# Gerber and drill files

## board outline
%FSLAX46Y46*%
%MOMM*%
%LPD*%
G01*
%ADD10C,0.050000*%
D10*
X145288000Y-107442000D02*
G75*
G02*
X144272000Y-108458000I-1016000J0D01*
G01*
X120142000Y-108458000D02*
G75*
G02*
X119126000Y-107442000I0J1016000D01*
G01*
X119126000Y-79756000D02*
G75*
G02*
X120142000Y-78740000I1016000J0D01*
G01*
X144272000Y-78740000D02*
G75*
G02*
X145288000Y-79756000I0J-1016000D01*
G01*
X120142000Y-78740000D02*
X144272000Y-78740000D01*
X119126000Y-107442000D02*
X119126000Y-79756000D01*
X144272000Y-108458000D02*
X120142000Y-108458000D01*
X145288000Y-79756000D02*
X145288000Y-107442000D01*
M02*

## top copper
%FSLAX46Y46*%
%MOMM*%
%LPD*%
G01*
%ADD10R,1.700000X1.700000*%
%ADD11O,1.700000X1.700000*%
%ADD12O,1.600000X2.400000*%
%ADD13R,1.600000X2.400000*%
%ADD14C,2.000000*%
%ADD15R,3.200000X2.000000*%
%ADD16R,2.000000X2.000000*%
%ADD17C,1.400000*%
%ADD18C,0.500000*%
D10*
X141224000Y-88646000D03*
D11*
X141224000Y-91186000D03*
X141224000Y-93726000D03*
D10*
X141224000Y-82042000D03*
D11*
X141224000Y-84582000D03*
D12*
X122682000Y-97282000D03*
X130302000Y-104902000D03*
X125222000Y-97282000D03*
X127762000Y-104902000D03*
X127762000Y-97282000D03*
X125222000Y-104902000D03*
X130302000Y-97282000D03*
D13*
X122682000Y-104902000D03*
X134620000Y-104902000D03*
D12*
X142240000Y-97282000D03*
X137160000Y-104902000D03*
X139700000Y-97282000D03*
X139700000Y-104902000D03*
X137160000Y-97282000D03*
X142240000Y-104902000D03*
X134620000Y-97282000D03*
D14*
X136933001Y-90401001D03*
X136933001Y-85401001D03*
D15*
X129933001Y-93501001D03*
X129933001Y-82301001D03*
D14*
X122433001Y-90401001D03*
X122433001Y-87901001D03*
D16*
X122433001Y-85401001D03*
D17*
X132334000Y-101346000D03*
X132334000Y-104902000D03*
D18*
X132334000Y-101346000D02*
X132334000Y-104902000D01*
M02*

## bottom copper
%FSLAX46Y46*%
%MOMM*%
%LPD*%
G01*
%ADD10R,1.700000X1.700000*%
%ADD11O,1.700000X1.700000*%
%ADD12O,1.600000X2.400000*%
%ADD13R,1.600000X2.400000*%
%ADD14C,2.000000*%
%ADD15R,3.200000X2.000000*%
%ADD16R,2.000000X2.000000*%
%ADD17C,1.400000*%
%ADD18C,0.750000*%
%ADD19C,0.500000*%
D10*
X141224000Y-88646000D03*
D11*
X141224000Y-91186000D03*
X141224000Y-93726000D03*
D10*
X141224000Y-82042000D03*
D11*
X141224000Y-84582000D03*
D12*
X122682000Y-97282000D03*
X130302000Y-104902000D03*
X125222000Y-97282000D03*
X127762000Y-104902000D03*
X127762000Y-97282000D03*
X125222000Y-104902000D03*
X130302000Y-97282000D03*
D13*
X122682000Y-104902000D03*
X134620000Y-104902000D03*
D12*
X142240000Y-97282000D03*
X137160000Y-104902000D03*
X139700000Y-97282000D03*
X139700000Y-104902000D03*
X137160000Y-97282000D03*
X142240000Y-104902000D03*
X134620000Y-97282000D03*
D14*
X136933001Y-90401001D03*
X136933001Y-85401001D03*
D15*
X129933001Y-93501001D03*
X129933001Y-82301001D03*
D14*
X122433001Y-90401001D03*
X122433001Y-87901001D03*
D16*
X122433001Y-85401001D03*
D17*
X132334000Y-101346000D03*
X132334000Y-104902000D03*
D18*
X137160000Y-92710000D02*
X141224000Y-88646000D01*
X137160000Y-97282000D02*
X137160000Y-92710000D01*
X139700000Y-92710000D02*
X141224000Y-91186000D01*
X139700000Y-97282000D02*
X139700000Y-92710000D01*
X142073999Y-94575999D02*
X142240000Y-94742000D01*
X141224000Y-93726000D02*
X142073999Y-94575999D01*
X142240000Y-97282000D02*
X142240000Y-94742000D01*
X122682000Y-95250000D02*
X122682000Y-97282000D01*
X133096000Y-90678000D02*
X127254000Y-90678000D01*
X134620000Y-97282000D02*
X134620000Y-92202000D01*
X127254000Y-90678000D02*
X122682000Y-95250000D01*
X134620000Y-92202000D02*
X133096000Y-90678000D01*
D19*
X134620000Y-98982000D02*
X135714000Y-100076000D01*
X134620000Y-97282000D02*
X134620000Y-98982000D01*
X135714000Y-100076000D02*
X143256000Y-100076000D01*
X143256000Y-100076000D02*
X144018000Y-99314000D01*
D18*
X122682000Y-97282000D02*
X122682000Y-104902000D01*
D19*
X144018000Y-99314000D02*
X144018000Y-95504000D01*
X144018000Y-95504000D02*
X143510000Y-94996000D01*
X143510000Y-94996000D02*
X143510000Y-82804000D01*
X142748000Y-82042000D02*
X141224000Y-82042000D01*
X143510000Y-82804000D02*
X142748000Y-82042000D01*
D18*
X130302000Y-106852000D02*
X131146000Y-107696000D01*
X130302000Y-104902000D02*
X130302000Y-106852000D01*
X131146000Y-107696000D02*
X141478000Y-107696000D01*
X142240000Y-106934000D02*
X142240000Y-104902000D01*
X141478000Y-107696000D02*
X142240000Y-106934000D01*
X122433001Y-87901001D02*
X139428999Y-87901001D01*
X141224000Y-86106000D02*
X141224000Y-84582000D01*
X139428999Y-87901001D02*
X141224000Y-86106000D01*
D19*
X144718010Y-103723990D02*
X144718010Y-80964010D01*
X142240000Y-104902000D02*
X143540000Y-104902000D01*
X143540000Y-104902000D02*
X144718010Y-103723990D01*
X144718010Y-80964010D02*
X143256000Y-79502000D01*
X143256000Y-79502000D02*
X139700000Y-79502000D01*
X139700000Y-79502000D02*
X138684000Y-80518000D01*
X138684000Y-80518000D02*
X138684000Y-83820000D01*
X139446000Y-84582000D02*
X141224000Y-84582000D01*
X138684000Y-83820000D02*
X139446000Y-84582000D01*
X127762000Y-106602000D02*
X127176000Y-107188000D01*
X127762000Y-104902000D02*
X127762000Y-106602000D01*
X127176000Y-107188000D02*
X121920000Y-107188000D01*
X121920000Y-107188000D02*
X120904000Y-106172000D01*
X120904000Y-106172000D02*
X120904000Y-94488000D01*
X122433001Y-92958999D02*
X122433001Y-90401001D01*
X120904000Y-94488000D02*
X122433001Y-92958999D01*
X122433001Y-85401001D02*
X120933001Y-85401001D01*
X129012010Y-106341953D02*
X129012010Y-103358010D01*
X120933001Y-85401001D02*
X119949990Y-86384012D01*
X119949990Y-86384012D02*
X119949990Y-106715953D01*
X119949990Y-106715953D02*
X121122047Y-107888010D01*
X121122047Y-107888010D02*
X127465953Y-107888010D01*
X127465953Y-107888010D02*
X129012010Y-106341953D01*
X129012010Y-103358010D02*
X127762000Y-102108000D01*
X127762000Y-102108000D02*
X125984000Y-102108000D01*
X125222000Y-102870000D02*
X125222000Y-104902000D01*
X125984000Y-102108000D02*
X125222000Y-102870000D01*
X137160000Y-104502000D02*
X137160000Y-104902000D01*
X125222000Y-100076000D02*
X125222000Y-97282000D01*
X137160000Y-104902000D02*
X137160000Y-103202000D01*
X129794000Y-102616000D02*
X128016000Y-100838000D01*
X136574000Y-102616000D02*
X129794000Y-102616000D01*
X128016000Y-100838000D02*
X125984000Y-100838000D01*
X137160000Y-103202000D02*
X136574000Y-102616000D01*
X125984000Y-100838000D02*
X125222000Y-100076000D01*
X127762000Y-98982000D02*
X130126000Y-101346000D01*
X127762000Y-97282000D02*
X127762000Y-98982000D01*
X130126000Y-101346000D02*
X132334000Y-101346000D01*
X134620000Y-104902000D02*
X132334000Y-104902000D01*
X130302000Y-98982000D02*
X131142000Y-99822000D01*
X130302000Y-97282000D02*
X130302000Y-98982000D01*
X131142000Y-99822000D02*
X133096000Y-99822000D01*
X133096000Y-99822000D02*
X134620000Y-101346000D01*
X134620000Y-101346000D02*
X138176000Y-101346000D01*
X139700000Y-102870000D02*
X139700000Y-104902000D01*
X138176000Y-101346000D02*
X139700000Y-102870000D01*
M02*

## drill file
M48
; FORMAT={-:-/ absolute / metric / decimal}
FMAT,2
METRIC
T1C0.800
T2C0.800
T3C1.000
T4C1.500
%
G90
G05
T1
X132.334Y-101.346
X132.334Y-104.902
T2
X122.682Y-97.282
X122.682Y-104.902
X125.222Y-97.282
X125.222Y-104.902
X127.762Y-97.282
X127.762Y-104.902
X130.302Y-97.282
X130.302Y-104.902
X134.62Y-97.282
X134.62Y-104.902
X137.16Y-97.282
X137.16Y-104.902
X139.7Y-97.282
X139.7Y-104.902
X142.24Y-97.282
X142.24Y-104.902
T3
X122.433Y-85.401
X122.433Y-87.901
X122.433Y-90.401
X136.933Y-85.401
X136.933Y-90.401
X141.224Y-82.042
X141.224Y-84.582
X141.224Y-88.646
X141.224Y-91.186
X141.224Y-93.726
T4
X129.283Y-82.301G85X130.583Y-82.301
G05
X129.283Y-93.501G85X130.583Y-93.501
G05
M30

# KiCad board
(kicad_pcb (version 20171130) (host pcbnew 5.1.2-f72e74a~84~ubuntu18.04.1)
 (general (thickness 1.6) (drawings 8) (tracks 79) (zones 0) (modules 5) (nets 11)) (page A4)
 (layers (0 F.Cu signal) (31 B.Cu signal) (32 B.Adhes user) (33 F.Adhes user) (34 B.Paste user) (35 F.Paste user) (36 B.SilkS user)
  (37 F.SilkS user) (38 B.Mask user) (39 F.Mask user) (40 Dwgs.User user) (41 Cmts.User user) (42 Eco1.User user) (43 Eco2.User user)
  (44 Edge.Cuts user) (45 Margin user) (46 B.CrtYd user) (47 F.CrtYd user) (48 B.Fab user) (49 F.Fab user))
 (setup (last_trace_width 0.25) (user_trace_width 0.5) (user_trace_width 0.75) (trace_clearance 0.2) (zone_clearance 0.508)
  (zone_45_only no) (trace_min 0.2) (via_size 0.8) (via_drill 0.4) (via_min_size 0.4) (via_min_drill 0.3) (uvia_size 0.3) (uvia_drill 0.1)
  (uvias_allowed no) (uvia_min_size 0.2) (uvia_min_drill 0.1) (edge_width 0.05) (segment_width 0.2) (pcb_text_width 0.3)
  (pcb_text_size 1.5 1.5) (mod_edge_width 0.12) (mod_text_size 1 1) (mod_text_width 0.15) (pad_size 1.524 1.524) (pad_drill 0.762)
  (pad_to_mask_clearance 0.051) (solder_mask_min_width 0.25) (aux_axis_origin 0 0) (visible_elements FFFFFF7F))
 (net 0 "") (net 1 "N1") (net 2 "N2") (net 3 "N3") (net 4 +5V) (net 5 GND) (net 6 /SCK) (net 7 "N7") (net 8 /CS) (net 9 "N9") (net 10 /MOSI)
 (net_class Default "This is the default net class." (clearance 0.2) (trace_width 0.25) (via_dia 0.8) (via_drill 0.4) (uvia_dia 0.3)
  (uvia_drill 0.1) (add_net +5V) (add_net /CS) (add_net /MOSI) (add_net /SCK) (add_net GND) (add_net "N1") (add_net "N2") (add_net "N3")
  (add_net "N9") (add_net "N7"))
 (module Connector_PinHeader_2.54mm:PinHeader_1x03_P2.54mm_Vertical (layer F.Cu) (at 141.224 88.646)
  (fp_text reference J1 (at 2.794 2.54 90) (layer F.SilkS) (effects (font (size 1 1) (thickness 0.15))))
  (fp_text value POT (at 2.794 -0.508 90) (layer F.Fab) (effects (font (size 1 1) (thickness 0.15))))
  (pad 1 thru_hole rect (at 0 0) (size 1.7 1.7) (drill 1) (layers *.Cu *.Mask) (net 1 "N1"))
  (pad 2 thru_hole oval (at 0 2.54) (size 1.7 1.7) (drill 1) (layers *.Cu *.Mask) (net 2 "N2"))
  (pad 3 thru_hole oval (at 0 5.08) (size 1.7 1.7) (drill 1) (layers *.Cu *.Mask) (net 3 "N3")))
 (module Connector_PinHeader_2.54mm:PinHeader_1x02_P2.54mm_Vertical (layer F.Cu) (at 141.224 82.042)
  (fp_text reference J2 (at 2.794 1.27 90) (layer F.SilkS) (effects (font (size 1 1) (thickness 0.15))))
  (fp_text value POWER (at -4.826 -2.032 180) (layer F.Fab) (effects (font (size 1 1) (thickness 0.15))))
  (pad 1 thru_hole rect (at 0 0) (size 1.7 1.7) (drill 1) (layers *.Cu *.Mask) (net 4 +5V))
  (pad 2 thru_hole oval (at 0 2.54) (size 1.7 1.7) (drill 1) (layers *.Cu *.Mask) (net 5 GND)))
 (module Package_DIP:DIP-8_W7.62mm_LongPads (layer F.Cu) (at 122.682 104.902 90)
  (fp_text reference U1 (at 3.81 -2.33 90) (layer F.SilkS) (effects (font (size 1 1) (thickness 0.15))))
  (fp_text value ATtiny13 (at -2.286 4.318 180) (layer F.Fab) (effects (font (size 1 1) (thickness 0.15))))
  (pad 8 thru_hole oval (at 7.62 0 90) (size 2.4 1.6) (drill 0.8) (layers *.Cu *.Mask) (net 4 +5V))
  (pad 4 thru_hole oval (at 0 7.62 90) (size 2.4 1.6) (drill 0.8) (layers *.Cu *.Mask) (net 5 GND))
  (pad 7 thru_hole oval (at 7.62 2.54 90) (size 2.4 1.6) (drill 0.8) (layers *.Cu *.Mask) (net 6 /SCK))
  (pad 3 thru_hole oval (at 0 5.08 90) (size 2.4 1.6) (drill 0.8) (layers *.Cu *.Mask) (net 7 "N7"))
  (pad 6 thru_hole oval (at 7.62 5.08 90) (size 2.4 1.6) (drill 0.8) (layers *.Cu *.Mask) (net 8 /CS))
  (pad 2 thru_hole oval (at 0 2.54 90) (size 2.4 1.6) (drill 0.8) (layers *.Cu *.Mask) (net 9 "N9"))
  (pad 5 thru_hole oval (at 7.62 7.62 90) (size 2.4 1.6) (drill 0.8) (layers *.Cu *.Mask) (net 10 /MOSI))
  (pad 1 thru_hole rect (at 0 0 90) (size 2.4 1.6) (drill 0.8) (layers *.Cu *.Mask) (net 4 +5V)))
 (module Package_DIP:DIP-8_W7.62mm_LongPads (layer F.Cu) (at 134.62 104.902 90)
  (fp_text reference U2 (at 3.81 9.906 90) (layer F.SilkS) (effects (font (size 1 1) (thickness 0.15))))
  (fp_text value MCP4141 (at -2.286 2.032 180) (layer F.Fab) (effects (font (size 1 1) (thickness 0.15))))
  (pad 1 thru_hole rect (at 0 0 90) (size 2.4 1.6) (drill 0.8) (layers *.Cu *.Mask) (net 8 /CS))
  (pad 5 thru_hole oval (at 7.62 7.62 90) (size 2.4 1.6) (drill 0.8) (layers *.Cu *.Mask) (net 3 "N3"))
  (pad 2 thru_hole oval (at 0 2.54 90) (size 2.4 1.6) (drill 0.8) (layers *.Cu *.Mask) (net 6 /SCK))
  (pad 6 thru_hole oval (at 7.62 5.08 90) (size 2.4 1.6) (drill 0.8) (layers *.Cu *.Mask) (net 2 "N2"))
  (pad 3 thru_hole oval (at 0 5.08 90) (size 2.4 1.6) (drill 0.8) (layers *.Cu *.Mask) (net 10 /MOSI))
  (pad 7 thru_hole oval (at 7.62 2.54 90) (size 2.4 1.6) (drill 0.8) (layers *.Cu *.Mask) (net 1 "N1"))
  (pad 4 thru_hole oval (at 0 7.62 90) (size 2.4 1.6) (drill 0.8) (layers *.Cu *.Mask) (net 5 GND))
  (pad 8 thru_hole oval (at 7.62 0 90) (size 2.4 1.6) (drill 0.8) (layers *.Cu *.Mask) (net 4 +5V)))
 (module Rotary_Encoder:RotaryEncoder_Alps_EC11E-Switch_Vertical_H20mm (layer F.Cu) (at 122.433001 85.401001)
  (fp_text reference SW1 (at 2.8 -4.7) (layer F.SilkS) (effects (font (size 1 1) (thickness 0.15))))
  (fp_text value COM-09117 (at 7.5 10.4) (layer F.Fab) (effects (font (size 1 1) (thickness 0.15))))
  (pad S1 thru_hole circle (at 14.5 5) (size 2 2) (drill 1) (layers *.Cu *.Mask))
  (pad S2 thru_hole circle (at 14.5 0) (size 2 2) (drill 1) (layers *.Cu *.Mask))
  (pad MP thru_hole rect (at 7.5 8.1) (size 3.2 2) (drill oval 2.8 1.5) (layers *.Cu *.Mask))
  (pad MP thru_hole rect (at 7.5 -3.1) (size 3.2 2) (drill oval 2.8 1.5) (layers *.Cu *.Mask))
  (pad B thru_hole circle (at 0 5) (size 2 2) (drill 1) (layers *.Cu *.Mask) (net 7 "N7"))
  (pad C thru_hole circle (at 0 2.5) (size 2 2) (drill 1) (layers *.Cu *.Mask) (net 5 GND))
  (pad A thru_hole rect (at 0 0) (size 2 2) (drill 1) (layers *.Cu *.Mask) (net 9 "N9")))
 (gr_arc (start 144.272 107.442) (end 144.272 108.458) (angle -90) (layer Edge.Cuts) (width 0.05))
 (gr_arc (start 120.142 107.442) (end 119.126 107.442) (angle -90) (layer Edge.Cuts) (width 0.05))
 (gr_arc (start 120.142 79.756) (end 120.142 78.74) (angle -90) (layer Edge.Cuts) (width 0.05))
 (gr_arc (start 144.272 79.756) (end 145.288 79.756) (angle -90) (layer Edge.Cuts) (width 0.05))
 (gr_line (start 120.142 78.74) (end 144.272 78.74) (layer Edge.Cuts) (width 0.05))
 (gr_line (start 119.126 107.442) (end 119.126 79.756) (layer Edge.Cuts) (width 0.05))
 (gr_line (start 144.272 108.458) (end 120.142 108.458) (layer Edge.Cuts) (width 0.05))
 (gr_line (start 145.288 79.756) (end 145.288 107.442) (layer Edge.Cuts) (width 0.05))
 (segment (start 137.16 92.71) (end 141.224 88.646) (width 0.75) (layer B.Cu) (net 1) (status 20))
 (segment (start 137.16 97.282) (end 137.16 92.71) (width 0.75) (layer B.Cu) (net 1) (status 10))
 (segment (start 139.7 92.71) (end 141.224 91.186) (width 0.75) (layer B.Cu) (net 2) (status 20))
 (segment (start 139.7 97.282) (end 139.7 92.71) (width 0.75) (layer B.Cu) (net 2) (status 10))
 (segment (start 142.073999 94.575999) (end 142.24 94.742) (width 0.75) (layer B.Cu) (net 3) (status 10))
 (segment (start 141.224 93.726) (end 142.073999 94.575999) (width 0.75) (layer B.Cu) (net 3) (status 30))
 (segment (start 142.24 97.282) (end 142.24 94.742) (width 0.75) (layer B.Cu) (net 3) (status 10))
 (segment (start 122.682 95.25) (end 122.682 97.282) (width 0.75) (layer B.Cu) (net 4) (status 20))
 (segment (start 133.096 90.678) (end 127.254 90.678) (width 0.75) (layer B.Cu) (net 4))
 (segment (start 134.62 97.282) (end 134.62 92.202) (width 0.75) (layer B.Cu) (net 4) (status 10))
 (segment (start 127.254 90.678) (end 122.682 95.25) (width 0.75) (layer B.Cu) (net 4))
 (segment (start 134.62 92.202) (end 133.096 90.678) (width 0.75) (layer B.Cu) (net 4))
 (segment (start 134.62 98.982) (end 135.714 100.076) (width 0.5) (layer B.Cu) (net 4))
 (segment (start 134.62 97.282) (end 134.62 98.982) (width 0.5) (layer B.Cu) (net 4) (status 10))
 (segment (start 135.714 100.076) (end 143.256 100.076) (width 0.5) (layer B.Cu) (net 4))
 (segment (start 143.256 100.076) (end 144.018 99.314) (width 0.5) (layer B.Cu) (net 4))
 (segment (start 122.682 97.282) (end 122.682 104.902) (width 0.75) (layer B.Cu) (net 4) (status 30))
 (segment (start 144.018 99.314) (end 144.018 95.504) (width 0.5) (layer B.Cu) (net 4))
 (segment (start 144.018 95.504) (end 143.51 94.996) (width 0.5) (layer B.Cu) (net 4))
 (segment (start 143.51 94.996) (end 143.51 82.804) (width 0.5) (layer B.Cu) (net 4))
 (segment (start 142.748 82.042) (end 141.224 82.042) (width 0.5) (layer B.Cu) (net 4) (status 20))
 (segment (start 143.51 82.804) (end 142.748 82.042) (width 0.5) (layer B.Cu) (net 4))
 (segment (start 130.302 106.852) (end 131.146 107.696) (width 0.75) (layer B.Cu) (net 5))
 (segment (start 130.302 104.902) (end 130.302 106.852) (width 0.75) (layer B.Cu) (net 5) (status 10))
 (segment (start 131.146 107.696) (end 141.478 107.696) (width 0.75) (layer B.Cu) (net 5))
 (segment (start 142.24 106.934) (end 142.24 104.902) (width 0.75) (layer B.Cu) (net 5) (status 20))
 (segment (start 141.478 107.696) (end 142.24 106.934) (width 0.75) (layer B.Cu) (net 5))
 (segment (start 122.433001 87.901001) (end 139.428999 87.901001) (width 0.75) (layer B.Cu) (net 5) (status 10))
 (segment (start 141.224 86.106) (end 141.224 84.582) (width 0.75) (layer B.Cu) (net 5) (status 20))
 (segment (start 139.428999 87.901001) (end 141.224 86.106) (width 0.75) (layer B.Cu) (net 5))
 (segment (start 144.71801 103.72399) (end 144.71801 80.96401) (width 0.5) (layer B.Cu) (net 5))
 (segment (start 142.24 104.902) (end 143.54 104.902) (width 0.5) (layer B.Cu) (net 5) (status 10))
 (segment (start 143.54 104.902) (end 144.71801 103.72399) (width 0.5) (layer B.Cu) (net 5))
 (segment (start 144.71801 80.96401) (end 143.256 79.502) (width 0.5) (layer B.Cu) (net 5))
 (segment (start 143.256 79.502) (end 139.7 79.502) (width 0.5) (layer B.Cu) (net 5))
 (segment (start 139.7 79.502) (end 138.684 80.518) (width 0.5) (layer B.Cu) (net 5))
 (segment (start 138.684 80.518) (end 138.684 83.82) (width 0.5) (layer B.Cu) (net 5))
 (segment (start 139.446 84.582) (end 141.224 84.582) (width 0.5) (layer B.Cu) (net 5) (status 20))
 (segment (start 138.684 83.82) (end 139.446 84.582) (width 0.5) (layer B.Cu) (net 5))
 (segment (start 127.762 106.602) (end 127.176 107.188) (width 0.5) (layer B.Cu) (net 7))
 (segment (start 127.762 104.902) (end 127.762 106.602) (width 0.5) (layer B.Cu) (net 7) (status 10))
 (segment (start 127.176 107.188) (end 121.92 107.188) (width 0.5) (layer B.Cu) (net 7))
 (segment (start 121.92 107.188) (end 120.904 106.172) (width 0.5) (layer B.Cu) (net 7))
 (segment (start 120.904 106.172) (end 120.904 94.488) (width 0.5) (layer B.Cu) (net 7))
 (segment (start 122.433001 92.958999) (end 122.433001 90.401001) (width 0.5) (layer B.Cu) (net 7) (status 20))
 (segment (start 120.904 94.488) (end 122.433001 92.958999) (width 0.5) (layer B.Cu) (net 7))
 (segment (start 122.433001 85.401001) (end 120.933001 85.401001) (width 0.5) (layer B.Cu) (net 9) (status 10))
 (segment (start 129.01201 106.341953) (end 129.01201 103.35801) (width 0.5) (layer B.Cu) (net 9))
 (segment (start 120.933001 85.401001) (end 119.94999 86.384012) (width 0.5) (layer B.Cu) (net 9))
 (segment (start 119.94999 86.384012) (end 119.94999 106.715953) (width 0.5) (layer B.Cu) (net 9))
 (segment (start 119.94999 106.715953) (end 121.122047 107.88801) (width 0.5) (layer B.Cu) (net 9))
 (segment (start 121.122047 107.88801) (end 127.465953 107.88801) (width 0.5) (layer B.Cu) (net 9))
 (segment (start 127.465953 107.88801) (end 129.01201 106.341953) (width 0.5) (layer B.Cu) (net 9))
 (segment (start 129.01201 103.35801) (end 127.762 102.108) (width 0.5) (layer B.Cu) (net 9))
 (segment (start 127.762 102.108) (end 125.984 102.108) (width 0.5) (layer B.Cu) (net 9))
 (segment (start 125.222 102.87) (end 125.222 104.902) (width 0.5) (layer B.Cu) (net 9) (status 20))
 (segment (start 125.984 102.108) (end 125.222 102.87) (width 0.5) (layer B.Cu) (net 9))
 (segment (start 137.16 104.502) (end 137.16 104.902) (width 0.5) (layer B.Cu) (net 6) (status 30))
 (segment (start 125.222 100.076) (end 125.222 97.282) (width 0.5) (layer B.Cu) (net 6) (status 20))
 (segment (start 137.16 104.902) (end 137.16 103.202) (width 0.5) (layer B.Cu) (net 6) (status 10))
 (segment (start 129.794 102.616) (end 128.016 100.838) (width 0.5) (layer B.Cu) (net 6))
 (segment (start 136.574 102.616) (end 129.794 102.616) (width 0.5) (layer B.Cu) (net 6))
 (segment (start 128.016 100.838) (end 125.984 100.838) (width 0.5) (layer B.Cu) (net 6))
 (segment (start 137.16 103.202) (end 136.574 102.616) (width 0.5) (layer B.Cu) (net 6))
 (segment (start 125.984 100.838) (end 125.222 100.076) (width 0.5) (layer B.Cu) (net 6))
 (segment (start 127.762 98.982) (end 130.126 101.346) (width 0.5) (layer B.Cu) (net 8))
 (segment (start 127.762 97.282) (end 127.762 98.982) (width 0.5) (layer B.Cu) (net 8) (status 10))
 (segment (start 130.126 101.346) (end 132.334 101.346) (width 0.5) (layer B.Cu) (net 8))
 (via (at 132.334 101.346) (size 1.4) (drill 0.8) (layers F.Cu B.Cu) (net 8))
 (segment (start 134.62 104.902) (end 132.334 104.902) (width 0.5) (layer B.Cu) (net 8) (status 10))
 (via (at 132.334 104.902) (size 1.4) (drill 0.8) (layers F.Cu B.Cu) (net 8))
 (segment (start 132.334 101.346) (end 132.334 104.902) (width 0.5) (layer F.Cu) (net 8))
 (segment (start 130.302 98.982) (end 131.142 99.822) (width 0.5) (layer B.Cu) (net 10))
 (segment (start 130.302 97.282) (end 130.302 98.982) (width 0.5) (layer B.Cu) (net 10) (status 10))
 (segment (start 131.142 99.822) (end 133.096 99.822) (width 0.5) (layer B.Cu) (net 10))
 (segment (start 133.096 99.822) (end 134.62 101.346) (width 0.5) (layer B.Cu) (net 10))
 (segment (start 134.62 101.346) (end 138.176 101.346) (width 0.5) (layer B.Cu) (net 10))
 (segment (start 139.7 102.87) (end 139.7 104.902) (width 0.5) (layer B.Cu) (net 10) (status 20))
 (segment (start 138.176 101.346) (end 139.7 102.87) (width 0.5) (layer B.Cu) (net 10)))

